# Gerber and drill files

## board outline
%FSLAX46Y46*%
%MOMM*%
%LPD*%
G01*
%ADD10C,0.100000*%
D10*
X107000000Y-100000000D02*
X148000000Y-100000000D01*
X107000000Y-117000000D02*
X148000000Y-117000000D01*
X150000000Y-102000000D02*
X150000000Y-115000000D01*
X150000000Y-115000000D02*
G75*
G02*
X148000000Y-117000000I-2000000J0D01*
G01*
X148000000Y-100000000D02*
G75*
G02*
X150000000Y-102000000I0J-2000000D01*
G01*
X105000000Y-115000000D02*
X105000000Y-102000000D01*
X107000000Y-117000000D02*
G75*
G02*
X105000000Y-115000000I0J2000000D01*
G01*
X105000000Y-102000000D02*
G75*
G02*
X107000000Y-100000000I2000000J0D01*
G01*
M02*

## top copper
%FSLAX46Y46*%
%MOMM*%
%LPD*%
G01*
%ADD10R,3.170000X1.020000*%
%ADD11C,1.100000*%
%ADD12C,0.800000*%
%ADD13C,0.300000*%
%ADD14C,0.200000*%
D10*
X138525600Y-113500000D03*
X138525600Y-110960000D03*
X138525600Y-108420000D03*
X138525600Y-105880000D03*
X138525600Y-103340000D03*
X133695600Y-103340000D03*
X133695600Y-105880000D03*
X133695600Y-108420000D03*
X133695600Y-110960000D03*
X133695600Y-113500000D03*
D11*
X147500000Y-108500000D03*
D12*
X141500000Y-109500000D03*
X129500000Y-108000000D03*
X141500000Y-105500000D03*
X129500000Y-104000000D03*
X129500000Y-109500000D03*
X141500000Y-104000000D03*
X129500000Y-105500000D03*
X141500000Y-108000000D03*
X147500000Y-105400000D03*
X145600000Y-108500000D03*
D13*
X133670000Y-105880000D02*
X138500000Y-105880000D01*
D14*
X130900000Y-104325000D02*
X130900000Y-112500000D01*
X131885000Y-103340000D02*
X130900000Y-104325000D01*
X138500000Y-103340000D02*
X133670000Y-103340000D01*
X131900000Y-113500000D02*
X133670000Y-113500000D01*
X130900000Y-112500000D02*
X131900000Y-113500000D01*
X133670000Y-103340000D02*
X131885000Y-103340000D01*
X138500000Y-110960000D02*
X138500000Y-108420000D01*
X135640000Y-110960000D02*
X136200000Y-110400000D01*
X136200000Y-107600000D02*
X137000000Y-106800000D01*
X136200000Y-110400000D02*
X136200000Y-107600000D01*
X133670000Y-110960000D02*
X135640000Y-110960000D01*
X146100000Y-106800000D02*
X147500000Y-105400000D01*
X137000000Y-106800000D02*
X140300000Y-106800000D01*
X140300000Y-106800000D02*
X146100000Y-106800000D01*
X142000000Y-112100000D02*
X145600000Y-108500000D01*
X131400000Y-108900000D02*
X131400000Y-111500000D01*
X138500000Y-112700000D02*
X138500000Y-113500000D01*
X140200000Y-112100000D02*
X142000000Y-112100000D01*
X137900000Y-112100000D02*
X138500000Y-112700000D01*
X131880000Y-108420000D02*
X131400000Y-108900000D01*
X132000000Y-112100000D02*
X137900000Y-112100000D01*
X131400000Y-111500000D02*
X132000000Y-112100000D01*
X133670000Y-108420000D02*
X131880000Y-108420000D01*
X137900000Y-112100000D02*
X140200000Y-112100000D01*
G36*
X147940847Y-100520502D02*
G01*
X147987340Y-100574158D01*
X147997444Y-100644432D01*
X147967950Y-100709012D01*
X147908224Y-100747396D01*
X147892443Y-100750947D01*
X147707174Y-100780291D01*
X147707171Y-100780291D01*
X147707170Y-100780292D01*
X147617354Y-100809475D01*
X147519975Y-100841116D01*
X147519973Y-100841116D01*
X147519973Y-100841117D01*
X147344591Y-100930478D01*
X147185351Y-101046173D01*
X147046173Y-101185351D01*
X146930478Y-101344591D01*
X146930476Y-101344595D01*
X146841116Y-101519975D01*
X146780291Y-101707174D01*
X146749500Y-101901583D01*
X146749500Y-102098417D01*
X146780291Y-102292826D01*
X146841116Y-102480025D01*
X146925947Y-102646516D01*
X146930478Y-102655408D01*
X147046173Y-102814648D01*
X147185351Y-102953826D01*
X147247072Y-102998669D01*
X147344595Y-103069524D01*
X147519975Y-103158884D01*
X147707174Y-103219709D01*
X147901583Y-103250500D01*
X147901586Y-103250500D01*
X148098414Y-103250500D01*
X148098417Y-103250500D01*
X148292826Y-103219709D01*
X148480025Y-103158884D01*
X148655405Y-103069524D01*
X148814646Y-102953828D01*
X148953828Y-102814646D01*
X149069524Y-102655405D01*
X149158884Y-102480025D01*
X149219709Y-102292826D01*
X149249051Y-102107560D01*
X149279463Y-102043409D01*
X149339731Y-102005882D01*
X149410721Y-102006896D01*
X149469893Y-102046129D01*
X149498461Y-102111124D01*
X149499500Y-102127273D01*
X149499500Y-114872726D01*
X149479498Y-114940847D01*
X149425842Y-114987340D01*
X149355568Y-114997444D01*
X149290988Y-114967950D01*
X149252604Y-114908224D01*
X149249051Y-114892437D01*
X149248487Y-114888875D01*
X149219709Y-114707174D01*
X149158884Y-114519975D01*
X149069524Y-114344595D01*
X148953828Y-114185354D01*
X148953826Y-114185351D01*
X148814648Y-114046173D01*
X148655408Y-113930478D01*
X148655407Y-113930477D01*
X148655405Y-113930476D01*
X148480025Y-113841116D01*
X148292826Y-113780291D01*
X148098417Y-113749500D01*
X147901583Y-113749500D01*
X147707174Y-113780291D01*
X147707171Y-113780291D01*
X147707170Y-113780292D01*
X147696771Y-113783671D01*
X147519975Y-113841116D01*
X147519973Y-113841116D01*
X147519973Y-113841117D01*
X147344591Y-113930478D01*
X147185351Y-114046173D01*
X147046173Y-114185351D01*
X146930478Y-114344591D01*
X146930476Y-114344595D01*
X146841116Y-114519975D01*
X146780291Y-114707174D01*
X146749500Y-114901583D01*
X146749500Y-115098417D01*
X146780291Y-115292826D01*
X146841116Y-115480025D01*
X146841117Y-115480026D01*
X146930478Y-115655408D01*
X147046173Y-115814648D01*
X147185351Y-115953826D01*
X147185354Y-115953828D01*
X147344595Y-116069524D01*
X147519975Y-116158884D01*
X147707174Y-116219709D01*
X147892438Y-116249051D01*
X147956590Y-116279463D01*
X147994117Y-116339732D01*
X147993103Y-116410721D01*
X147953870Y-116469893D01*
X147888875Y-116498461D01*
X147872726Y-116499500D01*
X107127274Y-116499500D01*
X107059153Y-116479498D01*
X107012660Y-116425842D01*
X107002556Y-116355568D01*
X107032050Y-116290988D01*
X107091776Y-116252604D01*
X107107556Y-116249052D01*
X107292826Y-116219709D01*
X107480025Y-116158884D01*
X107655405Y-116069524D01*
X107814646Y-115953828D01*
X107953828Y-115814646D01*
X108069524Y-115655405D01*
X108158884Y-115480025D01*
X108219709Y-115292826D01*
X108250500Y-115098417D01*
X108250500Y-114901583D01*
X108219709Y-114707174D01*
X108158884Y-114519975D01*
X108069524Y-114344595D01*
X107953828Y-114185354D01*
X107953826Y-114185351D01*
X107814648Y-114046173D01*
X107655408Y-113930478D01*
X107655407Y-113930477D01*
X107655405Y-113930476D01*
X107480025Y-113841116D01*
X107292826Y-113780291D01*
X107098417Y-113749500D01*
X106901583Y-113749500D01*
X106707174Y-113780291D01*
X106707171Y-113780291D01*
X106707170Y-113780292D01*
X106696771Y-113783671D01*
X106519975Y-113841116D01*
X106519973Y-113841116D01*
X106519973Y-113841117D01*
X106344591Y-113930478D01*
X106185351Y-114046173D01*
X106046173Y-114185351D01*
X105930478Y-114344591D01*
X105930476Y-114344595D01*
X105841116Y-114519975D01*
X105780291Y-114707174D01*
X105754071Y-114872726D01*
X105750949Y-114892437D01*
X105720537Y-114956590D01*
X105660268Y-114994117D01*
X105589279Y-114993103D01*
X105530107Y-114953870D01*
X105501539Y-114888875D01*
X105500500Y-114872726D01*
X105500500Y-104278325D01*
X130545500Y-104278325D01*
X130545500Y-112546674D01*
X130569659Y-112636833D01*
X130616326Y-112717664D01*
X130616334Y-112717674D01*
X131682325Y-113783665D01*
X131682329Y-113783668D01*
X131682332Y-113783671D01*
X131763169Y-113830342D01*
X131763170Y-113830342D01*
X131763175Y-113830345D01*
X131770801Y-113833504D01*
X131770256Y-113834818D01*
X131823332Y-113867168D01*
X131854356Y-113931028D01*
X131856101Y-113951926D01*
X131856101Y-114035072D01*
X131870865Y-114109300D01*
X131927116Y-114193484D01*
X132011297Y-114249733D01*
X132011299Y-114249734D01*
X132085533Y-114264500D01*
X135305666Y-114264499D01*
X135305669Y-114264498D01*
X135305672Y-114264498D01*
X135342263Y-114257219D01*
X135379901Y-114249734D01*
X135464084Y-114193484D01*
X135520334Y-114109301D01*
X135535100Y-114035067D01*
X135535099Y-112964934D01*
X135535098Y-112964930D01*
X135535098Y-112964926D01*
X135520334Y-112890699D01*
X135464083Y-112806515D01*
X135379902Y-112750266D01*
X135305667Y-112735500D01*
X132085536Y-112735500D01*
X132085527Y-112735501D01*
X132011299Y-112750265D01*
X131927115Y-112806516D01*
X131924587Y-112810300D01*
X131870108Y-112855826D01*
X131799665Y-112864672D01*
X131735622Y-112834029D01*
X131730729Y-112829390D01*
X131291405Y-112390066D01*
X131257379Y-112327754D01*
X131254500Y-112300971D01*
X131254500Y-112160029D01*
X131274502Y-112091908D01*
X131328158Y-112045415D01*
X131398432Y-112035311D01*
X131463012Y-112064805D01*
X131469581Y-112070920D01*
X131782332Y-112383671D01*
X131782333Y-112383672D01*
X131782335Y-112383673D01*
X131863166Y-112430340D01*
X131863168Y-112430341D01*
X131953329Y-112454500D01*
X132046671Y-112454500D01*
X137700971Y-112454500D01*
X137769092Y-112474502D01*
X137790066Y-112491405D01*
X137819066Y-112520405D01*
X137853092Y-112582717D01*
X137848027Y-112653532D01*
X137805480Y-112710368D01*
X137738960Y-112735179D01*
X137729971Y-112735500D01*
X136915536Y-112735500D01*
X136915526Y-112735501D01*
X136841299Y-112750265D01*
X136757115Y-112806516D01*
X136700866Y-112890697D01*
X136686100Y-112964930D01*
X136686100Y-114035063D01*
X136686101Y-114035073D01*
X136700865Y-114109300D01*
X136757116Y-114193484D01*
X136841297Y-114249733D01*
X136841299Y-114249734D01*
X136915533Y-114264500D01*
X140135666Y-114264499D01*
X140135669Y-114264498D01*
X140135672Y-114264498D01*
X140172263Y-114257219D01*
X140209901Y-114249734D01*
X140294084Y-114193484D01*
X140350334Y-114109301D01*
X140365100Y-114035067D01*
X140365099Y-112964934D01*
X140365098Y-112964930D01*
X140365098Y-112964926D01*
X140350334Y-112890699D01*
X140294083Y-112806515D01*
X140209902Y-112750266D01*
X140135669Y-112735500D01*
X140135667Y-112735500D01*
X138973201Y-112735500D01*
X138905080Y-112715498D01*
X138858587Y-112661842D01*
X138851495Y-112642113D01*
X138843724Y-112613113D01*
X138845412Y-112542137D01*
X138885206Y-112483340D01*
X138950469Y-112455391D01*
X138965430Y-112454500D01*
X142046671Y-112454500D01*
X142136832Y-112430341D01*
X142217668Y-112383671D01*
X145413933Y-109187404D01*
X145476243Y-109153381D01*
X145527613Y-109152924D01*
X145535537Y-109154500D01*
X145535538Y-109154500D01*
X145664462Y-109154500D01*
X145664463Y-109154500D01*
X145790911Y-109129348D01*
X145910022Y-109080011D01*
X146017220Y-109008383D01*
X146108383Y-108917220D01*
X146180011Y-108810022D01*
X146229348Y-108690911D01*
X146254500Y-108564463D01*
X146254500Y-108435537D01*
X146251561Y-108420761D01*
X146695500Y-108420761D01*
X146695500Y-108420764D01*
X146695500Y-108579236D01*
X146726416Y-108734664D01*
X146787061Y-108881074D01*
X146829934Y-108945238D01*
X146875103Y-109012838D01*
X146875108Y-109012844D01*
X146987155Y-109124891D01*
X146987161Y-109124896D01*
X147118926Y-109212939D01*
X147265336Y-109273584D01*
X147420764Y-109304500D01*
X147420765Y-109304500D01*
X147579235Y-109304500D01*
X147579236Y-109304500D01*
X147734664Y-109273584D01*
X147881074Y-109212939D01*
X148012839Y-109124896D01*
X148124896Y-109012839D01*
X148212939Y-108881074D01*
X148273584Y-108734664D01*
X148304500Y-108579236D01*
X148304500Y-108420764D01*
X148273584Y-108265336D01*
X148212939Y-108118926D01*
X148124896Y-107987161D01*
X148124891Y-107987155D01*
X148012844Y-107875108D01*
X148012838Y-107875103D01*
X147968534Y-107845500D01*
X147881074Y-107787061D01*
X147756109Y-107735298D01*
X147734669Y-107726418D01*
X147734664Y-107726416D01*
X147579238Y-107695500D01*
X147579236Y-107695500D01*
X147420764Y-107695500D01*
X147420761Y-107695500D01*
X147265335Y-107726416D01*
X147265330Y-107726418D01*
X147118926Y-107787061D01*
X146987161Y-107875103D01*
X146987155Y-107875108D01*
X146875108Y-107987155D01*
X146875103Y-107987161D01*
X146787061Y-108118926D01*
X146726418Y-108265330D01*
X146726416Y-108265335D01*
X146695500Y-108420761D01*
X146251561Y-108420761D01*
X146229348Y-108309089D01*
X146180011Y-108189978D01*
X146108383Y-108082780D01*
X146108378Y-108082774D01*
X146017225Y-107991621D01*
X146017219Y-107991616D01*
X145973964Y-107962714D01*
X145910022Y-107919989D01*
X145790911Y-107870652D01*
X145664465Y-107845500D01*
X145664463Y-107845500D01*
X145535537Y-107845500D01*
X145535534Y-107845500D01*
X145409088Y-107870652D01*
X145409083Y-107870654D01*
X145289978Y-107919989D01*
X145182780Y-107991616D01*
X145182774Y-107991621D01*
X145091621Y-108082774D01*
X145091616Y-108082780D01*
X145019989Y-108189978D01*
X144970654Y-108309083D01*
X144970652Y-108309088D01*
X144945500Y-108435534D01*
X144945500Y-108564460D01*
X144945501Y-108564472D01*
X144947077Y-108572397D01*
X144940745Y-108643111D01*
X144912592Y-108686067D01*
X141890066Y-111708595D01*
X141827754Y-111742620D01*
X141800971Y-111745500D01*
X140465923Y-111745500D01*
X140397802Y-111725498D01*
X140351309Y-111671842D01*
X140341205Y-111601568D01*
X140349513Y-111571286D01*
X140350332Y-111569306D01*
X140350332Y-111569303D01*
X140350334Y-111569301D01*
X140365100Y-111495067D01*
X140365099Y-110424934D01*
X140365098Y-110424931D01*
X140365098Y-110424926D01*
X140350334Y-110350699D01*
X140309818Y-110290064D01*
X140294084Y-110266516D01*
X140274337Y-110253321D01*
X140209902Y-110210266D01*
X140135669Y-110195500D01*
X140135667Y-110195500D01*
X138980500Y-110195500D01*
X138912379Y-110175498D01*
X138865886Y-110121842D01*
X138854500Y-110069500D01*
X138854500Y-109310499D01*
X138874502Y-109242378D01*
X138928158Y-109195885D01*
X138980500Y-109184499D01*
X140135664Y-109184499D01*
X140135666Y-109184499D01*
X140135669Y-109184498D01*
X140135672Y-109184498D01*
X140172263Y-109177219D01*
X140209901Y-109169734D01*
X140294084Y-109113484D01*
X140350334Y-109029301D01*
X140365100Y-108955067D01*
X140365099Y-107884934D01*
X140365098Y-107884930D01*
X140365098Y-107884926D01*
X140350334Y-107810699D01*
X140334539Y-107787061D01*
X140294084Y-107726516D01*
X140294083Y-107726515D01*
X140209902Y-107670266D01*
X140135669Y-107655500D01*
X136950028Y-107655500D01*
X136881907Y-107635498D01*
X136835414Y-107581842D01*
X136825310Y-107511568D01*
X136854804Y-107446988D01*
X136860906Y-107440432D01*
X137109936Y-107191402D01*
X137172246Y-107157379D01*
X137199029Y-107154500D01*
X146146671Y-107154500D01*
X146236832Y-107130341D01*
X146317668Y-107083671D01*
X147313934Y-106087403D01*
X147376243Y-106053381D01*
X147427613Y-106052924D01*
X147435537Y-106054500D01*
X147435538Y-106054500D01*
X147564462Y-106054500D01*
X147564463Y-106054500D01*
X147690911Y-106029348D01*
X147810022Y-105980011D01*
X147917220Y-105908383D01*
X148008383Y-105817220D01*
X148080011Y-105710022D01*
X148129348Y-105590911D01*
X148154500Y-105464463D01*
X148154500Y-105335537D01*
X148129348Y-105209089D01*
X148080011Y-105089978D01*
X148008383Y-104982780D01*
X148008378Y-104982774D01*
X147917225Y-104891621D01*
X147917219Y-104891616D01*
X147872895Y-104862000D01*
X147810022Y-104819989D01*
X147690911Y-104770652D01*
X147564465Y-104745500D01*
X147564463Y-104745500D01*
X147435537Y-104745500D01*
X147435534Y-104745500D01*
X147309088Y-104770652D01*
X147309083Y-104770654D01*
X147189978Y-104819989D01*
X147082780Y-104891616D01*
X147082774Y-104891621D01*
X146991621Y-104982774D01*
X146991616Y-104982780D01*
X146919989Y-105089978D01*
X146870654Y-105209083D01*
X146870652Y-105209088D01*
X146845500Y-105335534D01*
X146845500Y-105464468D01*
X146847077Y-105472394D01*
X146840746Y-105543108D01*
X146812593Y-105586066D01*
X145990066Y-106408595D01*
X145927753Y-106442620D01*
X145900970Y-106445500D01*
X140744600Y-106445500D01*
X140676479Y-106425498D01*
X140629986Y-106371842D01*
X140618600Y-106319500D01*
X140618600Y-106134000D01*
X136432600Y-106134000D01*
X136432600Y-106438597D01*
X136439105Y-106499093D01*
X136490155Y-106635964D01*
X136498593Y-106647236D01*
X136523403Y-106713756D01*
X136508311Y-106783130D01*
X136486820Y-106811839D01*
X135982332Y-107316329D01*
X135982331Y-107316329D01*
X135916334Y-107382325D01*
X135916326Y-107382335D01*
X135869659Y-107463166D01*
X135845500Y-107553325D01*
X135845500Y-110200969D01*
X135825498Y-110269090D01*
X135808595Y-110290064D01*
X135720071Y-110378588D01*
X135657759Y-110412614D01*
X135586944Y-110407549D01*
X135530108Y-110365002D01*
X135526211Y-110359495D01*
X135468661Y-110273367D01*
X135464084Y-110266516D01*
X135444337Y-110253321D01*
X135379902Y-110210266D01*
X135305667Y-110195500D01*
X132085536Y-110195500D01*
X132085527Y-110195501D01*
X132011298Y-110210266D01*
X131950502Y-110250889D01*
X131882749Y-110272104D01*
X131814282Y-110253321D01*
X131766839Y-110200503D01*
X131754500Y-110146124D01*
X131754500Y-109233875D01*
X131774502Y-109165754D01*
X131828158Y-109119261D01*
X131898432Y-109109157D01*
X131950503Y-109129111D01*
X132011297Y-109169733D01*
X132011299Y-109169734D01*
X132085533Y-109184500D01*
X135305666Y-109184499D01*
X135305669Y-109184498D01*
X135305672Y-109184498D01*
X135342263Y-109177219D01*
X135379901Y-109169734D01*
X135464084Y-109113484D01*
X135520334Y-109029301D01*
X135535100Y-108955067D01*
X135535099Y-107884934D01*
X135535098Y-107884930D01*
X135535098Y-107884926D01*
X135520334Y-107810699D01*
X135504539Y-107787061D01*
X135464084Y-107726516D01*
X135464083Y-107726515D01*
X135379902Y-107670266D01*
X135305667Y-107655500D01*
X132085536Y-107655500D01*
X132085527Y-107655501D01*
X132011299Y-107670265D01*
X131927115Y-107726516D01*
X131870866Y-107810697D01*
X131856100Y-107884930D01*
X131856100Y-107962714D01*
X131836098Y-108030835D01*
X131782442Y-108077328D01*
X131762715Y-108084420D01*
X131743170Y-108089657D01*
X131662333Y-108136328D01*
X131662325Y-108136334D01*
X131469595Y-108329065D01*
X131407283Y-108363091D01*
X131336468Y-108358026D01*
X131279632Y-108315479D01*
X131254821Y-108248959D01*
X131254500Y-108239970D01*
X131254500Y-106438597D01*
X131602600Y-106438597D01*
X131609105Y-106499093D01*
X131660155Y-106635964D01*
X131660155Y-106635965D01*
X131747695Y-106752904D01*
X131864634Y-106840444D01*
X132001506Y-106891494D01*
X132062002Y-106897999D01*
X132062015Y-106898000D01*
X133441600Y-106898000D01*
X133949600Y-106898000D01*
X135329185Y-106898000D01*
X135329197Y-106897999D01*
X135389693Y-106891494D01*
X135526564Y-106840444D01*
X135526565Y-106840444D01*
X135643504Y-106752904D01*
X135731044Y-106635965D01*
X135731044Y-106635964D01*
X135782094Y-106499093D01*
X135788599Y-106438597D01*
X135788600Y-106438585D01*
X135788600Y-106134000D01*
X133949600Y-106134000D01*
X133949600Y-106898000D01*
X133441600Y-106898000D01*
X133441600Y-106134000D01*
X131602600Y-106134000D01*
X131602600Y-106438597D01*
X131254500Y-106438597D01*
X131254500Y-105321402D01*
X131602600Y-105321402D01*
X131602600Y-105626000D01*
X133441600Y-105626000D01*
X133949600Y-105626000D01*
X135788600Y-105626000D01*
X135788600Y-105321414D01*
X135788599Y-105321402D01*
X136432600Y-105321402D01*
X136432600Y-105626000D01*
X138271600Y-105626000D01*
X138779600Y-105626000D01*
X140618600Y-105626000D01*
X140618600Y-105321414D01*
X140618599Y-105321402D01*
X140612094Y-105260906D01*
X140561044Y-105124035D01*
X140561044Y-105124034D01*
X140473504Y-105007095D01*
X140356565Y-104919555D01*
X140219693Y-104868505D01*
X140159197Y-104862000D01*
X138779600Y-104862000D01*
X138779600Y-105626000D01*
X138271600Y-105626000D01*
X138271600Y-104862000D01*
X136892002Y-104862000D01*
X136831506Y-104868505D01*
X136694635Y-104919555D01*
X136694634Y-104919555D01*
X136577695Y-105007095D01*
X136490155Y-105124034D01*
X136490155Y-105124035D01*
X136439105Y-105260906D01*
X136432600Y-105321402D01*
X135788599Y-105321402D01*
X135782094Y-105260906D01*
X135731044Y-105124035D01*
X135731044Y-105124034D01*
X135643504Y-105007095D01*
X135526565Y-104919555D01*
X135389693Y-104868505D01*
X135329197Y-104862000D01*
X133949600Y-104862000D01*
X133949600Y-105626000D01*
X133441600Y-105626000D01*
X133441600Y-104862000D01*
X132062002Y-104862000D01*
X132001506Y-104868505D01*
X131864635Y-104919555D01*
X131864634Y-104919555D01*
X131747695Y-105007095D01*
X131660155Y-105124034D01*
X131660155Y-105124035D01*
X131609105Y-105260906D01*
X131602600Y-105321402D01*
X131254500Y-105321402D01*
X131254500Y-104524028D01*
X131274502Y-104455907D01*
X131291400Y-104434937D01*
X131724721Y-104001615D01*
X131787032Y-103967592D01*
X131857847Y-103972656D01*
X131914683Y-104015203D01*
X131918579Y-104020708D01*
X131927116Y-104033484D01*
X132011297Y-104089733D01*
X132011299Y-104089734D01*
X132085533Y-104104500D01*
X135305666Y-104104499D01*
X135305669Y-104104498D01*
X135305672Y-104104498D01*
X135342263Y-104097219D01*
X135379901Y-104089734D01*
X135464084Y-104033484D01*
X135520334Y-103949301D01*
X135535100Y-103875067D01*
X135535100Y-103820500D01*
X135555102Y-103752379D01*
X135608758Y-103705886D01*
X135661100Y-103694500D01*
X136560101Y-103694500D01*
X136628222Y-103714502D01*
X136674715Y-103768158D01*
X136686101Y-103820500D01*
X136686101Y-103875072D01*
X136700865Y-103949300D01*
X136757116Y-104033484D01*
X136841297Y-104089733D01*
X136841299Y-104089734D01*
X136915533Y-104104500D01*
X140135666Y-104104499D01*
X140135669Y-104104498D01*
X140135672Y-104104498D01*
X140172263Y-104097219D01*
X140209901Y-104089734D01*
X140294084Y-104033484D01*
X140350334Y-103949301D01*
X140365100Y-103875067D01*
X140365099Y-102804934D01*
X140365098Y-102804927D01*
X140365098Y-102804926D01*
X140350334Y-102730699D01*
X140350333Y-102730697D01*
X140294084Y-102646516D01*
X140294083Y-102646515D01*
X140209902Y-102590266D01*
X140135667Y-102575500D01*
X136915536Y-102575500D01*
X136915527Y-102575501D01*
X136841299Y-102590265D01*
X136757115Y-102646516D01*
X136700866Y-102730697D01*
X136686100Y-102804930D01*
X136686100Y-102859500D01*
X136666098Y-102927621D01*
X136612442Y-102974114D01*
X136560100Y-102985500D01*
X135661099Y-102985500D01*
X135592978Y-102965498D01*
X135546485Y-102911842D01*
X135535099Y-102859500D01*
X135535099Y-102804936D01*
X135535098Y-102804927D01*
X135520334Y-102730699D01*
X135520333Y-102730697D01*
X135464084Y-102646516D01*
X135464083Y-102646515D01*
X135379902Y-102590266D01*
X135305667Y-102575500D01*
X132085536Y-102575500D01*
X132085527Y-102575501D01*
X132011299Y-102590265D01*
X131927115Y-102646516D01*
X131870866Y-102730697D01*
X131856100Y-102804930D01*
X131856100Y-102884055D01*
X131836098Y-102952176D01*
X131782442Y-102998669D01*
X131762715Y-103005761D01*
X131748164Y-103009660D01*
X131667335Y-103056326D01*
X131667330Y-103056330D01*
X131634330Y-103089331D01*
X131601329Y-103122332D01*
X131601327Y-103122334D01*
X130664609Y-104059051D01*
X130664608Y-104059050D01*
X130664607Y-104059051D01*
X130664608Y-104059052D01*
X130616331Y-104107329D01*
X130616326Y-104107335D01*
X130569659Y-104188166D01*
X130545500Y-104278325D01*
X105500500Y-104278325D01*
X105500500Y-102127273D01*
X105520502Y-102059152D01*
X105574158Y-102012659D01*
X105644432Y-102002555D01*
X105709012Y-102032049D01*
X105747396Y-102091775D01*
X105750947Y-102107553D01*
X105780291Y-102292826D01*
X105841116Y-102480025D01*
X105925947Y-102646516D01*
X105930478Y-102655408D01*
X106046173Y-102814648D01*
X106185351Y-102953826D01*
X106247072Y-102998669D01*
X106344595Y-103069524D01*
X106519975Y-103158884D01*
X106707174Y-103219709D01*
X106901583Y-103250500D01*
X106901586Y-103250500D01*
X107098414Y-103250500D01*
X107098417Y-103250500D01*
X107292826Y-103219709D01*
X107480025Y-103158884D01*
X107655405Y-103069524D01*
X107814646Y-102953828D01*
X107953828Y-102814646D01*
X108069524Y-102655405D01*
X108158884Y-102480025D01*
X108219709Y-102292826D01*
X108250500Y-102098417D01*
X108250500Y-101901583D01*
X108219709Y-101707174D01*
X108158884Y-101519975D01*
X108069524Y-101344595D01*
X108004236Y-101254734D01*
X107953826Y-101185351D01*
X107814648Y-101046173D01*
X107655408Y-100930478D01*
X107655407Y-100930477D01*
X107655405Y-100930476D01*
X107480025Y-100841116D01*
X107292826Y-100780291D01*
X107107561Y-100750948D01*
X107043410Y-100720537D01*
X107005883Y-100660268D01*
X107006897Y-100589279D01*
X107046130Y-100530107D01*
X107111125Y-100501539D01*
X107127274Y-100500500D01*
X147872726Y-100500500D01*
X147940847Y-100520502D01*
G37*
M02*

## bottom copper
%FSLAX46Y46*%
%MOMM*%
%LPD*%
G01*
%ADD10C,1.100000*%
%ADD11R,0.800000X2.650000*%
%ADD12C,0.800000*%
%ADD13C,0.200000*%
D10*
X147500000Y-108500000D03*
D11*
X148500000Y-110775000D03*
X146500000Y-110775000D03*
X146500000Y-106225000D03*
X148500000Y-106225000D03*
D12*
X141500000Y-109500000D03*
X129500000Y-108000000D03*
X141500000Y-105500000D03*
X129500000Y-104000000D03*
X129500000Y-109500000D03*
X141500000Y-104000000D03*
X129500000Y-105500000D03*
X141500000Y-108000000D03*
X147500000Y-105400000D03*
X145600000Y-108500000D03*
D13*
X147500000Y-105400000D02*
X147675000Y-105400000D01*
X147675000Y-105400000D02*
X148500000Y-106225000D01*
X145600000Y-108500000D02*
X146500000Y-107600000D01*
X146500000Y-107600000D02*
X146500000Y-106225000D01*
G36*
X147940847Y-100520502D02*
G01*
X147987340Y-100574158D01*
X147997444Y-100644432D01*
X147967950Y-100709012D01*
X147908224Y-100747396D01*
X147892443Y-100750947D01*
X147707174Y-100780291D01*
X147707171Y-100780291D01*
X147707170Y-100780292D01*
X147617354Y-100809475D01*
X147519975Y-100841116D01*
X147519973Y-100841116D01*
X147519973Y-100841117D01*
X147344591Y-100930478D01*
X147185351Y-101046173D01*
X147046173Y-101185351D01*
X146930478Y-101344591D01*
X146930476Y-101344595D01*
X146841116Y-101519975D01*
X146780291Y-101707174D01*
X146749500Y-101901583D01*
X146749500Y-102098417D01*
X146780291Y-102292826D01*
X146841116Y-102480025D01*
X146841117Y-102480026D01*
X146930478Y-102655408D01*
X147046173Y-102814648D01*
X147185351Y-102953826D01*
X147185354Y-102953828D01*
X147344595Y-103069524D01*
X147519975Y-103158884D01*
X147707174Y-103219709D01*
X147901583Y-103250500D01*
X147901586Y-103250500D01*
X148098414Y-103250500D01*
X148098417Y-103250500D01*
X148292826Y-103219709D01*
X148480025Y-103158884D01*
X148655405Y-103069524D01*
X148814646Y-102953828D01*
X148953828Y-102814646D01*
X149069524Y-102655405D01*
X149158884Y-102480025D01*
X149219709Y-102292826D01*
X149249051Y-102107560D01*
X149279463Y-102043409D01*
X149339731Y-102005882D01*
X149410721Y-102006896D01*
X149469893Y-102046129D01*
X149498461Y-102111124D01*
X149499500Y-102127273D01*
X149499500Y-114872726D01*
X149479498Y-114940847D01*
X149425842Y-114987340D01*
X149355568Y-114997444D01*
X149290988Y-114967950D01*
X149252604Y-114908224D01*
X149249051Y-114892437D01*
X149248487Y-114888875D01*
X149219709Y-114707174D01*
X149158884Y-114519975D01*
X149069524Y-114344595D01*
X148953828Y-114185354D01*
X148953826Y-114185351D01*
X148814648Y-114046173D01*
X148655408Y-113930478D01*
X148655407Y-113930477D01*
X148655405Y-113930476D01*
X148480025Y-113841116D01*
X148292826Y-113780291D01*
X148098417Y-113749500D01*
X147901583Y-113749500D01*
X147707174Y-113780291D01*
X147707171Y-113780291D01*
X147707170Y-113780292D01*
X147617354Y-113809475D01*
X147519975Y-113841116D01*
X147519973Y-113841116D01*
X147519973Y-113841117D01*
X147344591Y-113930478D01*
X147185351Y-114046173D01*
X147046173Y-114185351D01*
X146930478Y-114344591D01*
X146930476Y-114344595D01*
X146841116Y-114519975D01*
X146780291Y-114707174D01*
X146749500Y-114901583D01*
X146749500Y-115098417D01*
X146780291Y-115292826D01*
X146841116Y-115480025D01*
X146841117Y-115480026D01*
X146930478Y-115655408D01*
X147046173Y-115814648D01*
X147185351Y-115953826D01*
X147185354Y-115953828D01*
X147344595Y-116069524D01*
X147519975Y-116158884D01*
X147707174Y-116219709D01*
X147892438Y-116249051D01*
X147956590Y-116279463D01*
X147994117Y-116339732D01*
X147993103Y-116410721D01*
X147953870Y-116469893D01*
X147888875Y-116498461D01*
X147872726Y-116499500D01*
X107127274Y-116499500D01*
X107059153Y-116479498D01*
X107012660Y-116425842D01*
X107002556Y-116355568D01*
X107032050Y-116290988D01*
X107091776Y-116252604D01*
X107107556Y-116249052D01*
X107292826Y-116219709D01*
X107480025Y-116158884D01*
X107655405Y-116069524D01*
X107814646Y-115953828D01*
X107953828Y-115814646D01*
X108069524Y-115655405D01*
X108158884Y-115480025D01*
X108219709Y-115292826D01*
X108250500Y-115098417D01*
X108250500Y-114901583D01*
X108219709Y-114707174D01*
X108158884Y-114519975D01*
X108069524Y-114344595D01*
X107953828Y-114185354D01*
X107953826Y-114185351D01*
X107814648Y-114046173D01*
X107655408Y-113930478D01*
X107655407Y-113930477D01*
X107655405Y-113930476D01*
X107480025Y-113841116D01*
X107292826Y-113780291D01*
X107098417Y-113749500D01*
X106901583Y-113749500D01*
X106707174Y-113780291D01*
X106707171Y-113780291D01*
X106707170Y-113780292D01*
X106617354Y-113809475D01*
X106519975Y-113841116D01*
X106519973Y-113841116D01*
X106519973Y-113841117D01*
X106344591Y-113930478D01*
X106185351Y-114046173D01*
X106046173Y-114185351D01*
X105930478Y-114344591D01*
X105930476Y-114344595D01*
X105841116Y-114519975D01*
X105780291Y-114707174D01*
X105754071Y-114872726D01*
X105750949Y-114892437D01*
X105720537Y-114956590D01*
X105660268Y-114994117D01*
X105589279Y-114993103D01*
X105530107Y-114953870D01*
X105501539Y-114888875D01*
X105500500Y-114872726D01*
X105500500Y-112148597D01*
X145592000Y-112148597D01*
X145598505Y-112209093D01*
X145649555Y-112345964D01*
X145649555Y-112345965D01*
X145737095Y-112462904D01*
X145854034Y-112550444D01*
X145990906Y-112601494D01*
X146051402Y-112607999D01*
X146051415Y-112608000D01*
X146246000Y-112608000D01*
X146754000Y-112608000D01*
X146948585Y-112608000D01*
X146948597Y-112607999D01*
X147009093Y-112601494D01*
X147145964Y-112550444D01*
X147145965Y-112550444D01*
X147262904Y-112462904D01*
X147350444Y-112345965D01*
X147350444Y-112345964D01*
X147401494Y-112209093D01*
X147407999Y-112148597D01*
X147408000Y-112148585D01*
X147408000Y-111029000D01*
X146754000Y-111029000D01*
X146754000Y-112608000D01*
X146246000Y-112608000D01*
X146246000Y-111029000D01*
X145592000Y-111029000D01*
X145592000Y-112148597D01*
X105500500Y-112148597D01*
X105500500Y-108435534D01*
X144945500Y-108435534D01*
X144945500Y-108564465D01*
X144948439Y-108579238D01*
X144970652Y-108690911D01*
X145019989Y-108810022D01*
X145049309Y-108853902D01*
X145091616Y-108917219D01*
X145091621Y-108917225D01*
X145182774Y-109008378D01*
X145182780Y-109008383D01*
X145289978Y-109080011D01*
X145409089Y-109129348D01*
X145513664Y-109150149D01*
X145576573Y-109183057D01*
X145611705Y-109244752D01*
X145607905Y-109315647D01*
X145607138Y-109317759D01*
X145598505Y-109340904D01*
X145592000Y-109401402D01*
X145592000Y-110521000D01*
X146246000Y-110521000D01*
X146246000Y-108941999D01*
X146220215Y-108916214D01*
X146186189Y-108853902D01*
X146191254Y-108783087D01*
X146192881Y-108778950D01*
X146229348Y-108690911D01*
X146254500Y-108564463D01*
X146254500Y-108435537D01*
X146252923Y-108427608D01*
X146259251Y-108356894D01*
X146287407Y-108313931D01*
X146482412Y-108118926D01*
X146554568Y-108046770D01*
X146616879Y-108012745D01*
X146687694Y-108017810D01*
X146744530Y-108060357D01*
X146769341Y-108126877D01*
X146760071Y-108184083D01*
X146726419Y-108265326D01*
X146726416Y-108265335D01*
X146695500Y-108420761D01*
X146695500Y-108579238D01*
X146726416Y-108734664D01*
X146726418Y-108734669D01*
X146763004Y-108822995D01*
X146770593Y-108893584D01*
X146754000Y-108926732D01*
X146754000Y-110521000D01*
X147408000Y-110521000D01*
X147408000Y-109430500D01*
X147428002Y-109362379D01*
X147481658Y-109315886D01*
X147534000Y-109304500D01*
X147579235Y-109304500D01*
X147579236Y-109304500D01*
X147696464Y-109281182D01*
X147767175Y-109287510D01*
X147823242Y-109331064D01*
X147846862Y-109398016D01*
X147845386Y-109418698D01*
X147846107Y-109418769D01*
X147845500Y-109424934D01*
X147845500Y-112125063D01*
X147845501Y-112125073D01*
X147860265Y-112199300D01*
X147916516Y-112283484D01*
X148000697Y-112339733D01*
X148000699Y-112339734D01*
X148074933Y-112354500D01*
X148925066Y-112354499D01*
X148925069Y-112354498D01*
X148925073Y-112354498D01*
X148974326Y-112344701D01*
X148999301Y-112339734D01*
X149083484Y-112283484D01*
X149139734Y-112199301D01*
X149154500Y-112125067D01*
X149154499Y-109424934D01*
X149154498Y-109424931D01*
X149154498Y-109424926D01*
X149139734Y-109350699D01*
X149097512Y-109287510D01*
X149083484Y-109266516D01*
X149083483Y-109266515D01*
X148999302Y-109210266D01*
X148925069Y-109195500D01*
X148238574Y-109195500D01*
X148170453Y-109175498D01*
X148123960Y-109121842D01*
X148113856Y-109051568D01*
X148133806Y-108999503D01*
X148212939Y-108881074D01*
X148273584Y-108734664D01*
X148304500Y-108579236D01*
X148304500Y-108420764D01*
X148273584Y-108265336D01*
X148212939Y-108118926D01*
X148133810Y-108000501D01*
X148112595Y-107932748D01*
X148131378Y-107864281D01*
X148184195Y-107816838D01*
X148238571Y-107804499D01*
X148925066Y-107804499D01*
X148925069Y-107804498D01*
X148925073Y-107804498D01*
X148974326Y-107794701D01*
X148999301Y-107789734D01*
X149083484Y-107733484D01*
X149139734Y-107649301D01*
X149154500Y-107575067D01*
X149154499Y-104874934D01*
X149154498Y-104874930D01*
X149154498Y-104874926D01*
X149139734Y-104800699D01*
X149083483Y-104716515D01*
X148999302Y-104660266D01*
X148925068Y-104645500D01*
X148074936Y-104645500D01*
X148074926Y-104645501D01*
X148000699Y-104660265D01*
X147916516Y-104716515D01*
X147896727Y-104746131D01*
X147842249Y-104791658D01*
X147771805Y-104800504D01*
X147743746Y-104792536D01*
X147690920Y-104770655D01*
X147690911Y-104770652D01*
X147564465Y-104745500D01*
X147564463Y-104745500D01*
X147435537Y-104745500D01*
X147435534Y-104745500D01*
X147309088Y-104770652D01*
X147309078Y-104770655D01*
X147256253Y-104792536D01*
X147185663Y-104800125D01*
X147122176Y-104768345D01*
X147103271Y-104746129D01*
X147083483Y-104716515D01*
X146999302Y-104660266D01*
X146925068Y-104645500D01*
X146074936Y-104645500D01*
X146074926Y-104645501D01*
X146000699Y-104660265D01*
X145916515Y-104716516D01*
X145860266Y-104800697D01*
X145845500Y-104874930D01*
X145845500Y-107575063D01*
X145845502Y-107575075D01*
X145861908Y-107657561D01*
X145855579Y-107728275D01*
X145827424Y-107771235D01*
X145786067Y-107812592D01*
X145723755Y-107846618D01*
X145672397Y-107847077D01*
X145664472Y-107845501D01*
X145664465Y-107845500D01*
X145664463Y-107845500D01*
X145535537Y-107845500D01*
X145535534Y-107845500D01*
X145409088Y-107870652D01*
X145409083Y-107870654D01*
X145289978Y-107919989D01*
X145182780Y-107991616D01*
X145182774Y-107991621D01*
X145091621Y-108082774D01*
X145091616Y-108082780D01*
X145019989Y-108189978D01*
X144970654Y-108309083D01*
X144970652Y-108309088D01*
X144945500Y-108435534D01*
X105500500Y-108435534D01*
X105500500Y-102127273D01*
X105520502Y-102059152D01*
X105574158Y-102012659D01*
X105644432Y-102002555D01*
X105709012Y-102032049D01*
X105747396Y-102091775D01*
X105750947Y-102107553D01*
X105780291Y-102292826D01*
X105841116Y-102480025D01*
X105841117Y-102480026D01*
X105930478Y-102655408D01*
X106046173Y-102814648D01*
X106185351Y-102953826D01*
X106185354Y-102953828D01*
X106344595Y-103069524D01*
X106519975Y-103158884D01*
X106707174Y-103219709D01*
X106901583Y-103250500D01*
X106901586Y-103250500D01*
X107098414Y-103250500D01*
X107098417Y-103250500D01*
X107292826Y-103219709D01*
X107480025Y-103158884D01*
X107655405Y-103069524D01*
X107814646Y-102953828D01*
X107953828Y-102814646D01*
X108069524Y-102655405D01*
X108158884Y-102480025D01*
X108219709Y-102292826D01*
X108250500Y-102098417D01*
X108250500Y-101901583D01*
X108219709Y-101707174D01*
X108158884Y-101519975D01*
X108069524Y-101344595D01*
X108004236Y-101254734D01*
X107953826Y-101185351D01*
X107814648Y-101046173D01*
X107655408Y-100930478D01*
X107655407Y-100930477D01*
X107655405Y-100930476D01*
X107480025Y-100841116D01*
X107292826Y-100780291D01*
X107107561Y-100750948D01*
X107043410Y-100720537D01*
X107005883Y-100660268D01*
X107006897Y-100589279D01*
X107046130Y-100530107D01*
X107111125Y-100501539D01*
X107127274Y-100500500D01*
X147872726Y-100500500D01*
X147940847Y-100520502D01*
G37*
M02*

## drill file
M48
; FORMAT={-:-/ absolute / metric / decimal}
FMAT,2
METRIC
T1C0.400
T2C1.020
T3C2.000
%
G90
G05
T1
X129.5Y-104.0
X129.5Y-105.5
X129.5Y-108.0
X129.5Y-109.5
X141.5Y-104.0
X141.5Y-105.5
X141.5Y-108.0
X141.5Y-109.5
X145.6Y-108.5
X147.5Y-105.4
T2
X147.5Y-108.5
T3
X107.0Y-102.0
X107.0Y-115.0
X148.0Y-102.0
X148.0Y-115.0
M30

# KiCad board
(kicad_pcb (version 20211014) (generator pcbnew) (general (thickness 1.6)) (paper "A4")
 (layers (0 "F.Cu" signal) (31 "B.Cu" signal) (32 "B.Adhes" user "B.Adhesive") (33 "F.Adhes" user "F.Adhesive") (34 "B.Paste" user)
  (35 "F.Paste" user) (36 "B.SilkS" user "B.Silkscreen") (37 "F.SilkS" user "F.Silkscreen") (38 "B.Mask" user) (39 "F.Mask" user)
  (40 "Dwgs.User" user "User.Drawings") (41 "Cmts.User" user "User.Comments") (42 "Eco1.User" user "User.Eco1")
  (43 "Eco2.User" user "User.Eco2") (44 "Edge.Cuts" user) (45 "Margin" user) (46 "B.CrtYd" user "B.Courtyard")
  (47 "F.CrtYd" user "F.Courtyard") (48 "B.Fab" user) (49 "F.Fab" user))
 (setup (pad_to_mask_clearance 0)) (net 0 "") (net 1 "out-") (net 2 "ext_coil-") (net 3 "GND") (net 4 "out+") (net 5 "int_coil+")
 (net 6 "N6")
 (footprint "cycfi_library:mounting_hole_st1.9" (layer "F.Cu") (at 107 102)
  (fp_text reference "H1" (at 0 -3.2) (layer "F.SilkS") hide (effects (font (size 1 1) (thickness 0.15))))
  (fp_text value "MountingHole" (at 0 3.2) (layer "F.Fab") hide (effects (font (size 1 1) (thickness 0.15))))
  (pad "" np_thru_hole circle locked (at 0 0) (size 2 2) (drill 2) (layers *.Cu *.Mask)))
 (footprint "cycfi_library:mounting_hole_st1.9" (layer "F.Cu") (at 107 115)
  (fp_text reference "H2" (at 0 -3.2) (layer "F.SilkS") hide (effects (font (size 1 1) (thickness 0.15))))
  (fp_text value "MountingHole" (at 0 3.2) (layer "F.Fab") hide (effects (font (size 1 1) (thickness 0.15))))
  (pad "" np_thru_hole circle locked (at 0 0) (size 2 2) (drill 2) (layers *.Cu *.Mask)))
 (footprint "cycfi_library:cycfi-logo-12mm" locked (layer "F.Cu") (at 109.75 108.5 -90)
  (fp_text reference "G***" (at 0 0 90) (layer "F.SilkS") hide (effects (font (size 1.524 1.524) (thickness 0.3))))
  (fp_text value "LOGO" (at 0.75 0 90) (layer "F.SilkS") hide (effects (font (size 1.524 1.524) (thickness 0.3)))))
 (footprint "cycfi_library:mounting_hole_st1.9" (layer "F.Cu") (at 148 102)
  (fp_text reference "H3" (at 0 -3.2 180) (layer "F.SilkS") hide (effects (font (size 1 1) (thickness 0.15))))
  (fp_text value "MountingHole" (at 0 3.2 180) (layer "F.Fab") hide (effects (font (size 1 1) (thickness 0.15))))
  (pad "" np_thru_hole circle locked (at 0 0) (size 2 2) (drill 2) (layers *.Cu *.Mask)))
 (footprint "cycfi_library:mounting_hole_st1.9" (layer "F.Cu") (at 148 115)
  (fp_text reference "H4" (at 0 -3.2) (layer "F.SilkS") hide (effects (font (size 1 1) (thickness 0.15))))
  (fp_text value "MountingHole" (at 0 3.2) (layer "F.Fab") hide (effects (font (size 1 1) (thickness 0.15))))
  (pad "" np_thru_hole circle locked (at 0 0) (size 2 2) (drill 2) (layers *.Cu *.Mask)))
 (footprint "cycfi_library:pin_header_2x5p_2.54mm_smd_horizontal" (layer "F.Cu") (at 136.1 108.42 180)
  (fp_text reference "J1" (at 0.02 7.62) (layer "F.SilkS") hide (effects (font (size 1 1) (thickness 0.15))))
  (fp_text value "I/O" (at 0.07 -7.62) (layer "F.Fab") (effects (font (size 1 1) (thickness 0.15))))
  (pad "1" smd rect (at -2.4256 -5.08 180) (size 3.17 1.02) (layers "F.Cu" "F.Paste" "F.Mask") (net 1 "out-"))
  (pad "2" smd rect (at -2.4256 -2.54 180) (size 3.17 1.02) (layers "F.Cu" "F.Paste" "F.Mask") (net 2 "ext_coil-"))
  (pad "3" smd rect (at -2.4256 0 180) (size 3.17 1.02) (layers "F.Cu" "F.Paste" "F.Mask") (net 2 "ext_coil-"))
  (pad "4" smd rect (at -2.4256 2.54 180) (size 3.17 1.02) (layers "F.Cu" "F.Paste" "F.Mask") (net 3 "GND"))
  (pad "5" smd rect (at -2.4256 5.08 180) (size 3.17 1.02) (layers "F.Cu" "F.Paste" "F.Mask") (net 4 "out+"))
  (pad "6" smd rect (at 2.4044 5.08 180) (size 3.17 1.02) (layers "F.Cu" "F.Paste" "F.Mask") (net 4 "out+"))
  (pad "7" smd rect (at 2.4044 2.54 180) (size 3.17 1.02) (layers "F.Cu" "F.Paste" "F.Mask") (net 3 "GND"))
  (pad "8" smd rect (at 2.4044 0 180) (size 3.17 1.02) (layers "F.Cu" "F.Paste" "F.Mask") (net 1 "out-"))
  (pad "9" smd rect (at 2.4044 -2.54 180) (size 3.17 1.02) (layers "F.Cu" "F.Paste" "F.Mask") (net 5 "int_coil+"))
  (pad "10" smd rect (at 2.4044 -5.08 180) (size 3.17 1.02) (layers "F.Cu" "F.Paste" "F.Mask") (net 4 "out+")))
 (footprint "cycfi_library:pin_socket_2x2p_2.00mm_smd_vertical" (layer "B.Cu") (at 147.5 108.5 90)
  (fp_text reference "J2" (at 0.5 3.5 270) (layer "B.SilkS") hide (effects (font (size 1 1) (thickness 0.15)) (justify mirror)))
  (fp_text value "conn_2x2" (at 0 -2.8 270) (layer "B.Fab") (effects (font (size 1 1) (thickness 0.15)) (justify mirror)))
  (pad "" np_thru_hole circle (at 0 0 90) (size 1.1 1.1) (drill 1.02) (layers F&B.Cu *.Mask))
  (pad "1" smd rect (at -2.275 1 90) (size 2.65 0.8) (layers "B.Cu" "B.Paste" "B.Mask") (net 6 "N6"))
  (pad "2" smd rect (at -2.275 -1 90) (size 2.65 0.8) (layers "B.Cu" "B.Paste" "B.Mask") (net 3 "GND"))
  (pad "3" smd rect (at 2.275 -1 90) (size 2.65 0.8) (layers "B.Cu" "B.Paste" "B.Mask") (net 1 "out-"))
  (pad "4" smd rect (at 2.275 1 90) (size 2.65 0.8) (layers "B.Cu" "B.Paste" "B.Mask") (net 5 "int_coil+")))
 (gr_line (start 107 100) (end 148 100) (layer "Edge.Cuts") (width 0.1))
 (gr_line (start 107 117) (end 148 117) (layer "Edge.Cuts") (width 0.1))
 (gr_line (start 150 102) (end 150 115) (layer "Edge.Cuts") (width 0.1))
 (gr_arc (start 150 115) (mid 149.414214 116.414214) (end 148 117) (layer "Edge.Cuts") (width 0.1))
 (gr_arc (start 148 100) (mid 149.414214 100.585786) (end 150 102) (layer "Edge.Cuts") (width 0.1))
 (gr_line (start 105 115) (end 105 102) (layer "Edge.Cuts") (width 0.1))
 (gr_arc (start 107 117) (mid 105.585786 116.414214) (end 105 115) (layer "Edge.Cuts") (width 0.1))
 (gr_arc (start 105 102) (mid 105.585786 100.585786) (end 107 100) (layer "Edge.Cuts") (width 0.1))
 (segment (start 133.67 105.88) (end 138.5 105.88) (width 0.3) (layer "F.Cu") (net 3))
 (via (at 141.5 109.5) (size 0.8) (drill 0.4) (layers "F.Cu" "B.Cu") (free) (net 3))
 (via (at 129.5 108) (size 0.8) (drill 0.4) (layers "F.Cu" "B.Cu") (free) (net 3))
 (via (at 141.5 105.5) (size 0.8) (drill 0.4) (layers "F.Cu" "B.Cu") (free) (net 3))
 (via (at 129.5 104) (size 0.8) (drill 0.4) (layers "F.Cu" "B.Cu") (free) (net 3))
 (via (at 129.5 109.5) (size 0.8) (drill 0.4) (layers "F.Cu" "B.Cu") (free) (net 3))
 (via (at 141.5 104) (size 0.8) (drill 0.4) (layers "F.Cu" "B.Cu") (free) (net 3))
 (via (at 129.5 105.5) (size 0.8) (drill 0.4) (layers "F.Cu" "B.Cu") (free) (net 3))
 (via (at 141.5 108) (size 0.8) (drill 0.4) (layers "F.Cu" "B.Cu") (free) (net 3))
 (segment (start 130.9 104.325) (end 130.9 112.5) (width 0.2) (layer "F.Cu") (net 4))
 (segment (start 131.885 103.34) (end 130.9 104.325) (width 0.2) (layer "F.Cu") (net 4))
 (segment (start 138.5 103.34) (end 133.67 103.34) (width 0.2) (layer "F.Cu") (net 4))
 (segment (start 131.9 113.5) (end 133.67 113.5) (width 0.2) (layer "F.Cu") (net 4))
 (segment (start 130.9 112.5) (end 131.9 113.5) (width 0.2) (layer "F.Cu") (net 4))
 (segment (start 133.67 103.34) (end 131.885 103.34) (width 0.2) (layer "F.Cu") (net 4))
 (segment (start 138.5 110.96) (end 138.5 108.42) (width 0.2) (layer "F.Cu") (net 2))
 (segment (start 135.64 110.96) (end 136.2 110.4) (width 0.2) (layer "F.Cu") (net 5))
 (segment (start 136.2 107.6) (end 137 106.8) (width 0.2) (layer "F.Cu") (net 5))
 (segment (start 136.2 110.4) (end 136.2 107.6) (width 0.2) (layer "F.Cu") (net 5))
 (segment (start 133.67 110.96) (end 135.64 110.96) (width 0.2) (layer "F.Cu") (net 5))
 (segment (start 146.1 106.8) (end 147.5 105.4) (width 0.2) (layer "F.Cu") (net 5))
 (segment (start 137 106.8) (end 140.3 106.8) (width 0.2) (layer "F.Cu") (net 5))
 (segment (start 140.3 106.8) (end 146.1 106.8) (width 0.2) (layer "F.Cu") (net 5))
 (via (at 147.5 105.4) (size 0.8) (drill 0.4) (layers "F.Cu" "B.Cu") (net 5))
 (segment (start 147.5 105.4) (end 147.675 105.4) (width 0.2) (layer "B.Cu") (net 5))
 (segment (start 147.675 105.4) (end 148.5 106.225) (width 0.2) (layer "B.Cu") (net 5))
 (segment (start 142 112.1) (end 145.6 108.5) (width 0.2) (layer "F.Cu") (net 1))
 (segment (start 131.4 108.9) (end 131.4 111.5) (width 0.2) (layer "F.Cu") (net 1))
 (segment (start 138.5 112.7) (end 138.5 113.5) (width 0.2) (layer "F.Cu") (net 1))
 (segment (start 140.2 112.1) (end 142 112.1) (width 0.2) (layer "F.Cu") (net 1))
 (segment (start 137.9 112.1) (end 138.5 112.7) (width 0.2) (layer "F.Cu") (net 1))
 (segment (start 131.88 108.42) (end 131.4 108.9) (width 0.2) (layer "F.Cu") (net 1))
 (segment (start 132 112.1) (end 137.9 112.1) (width 0.2) (layer "F.Cu") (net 1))
 (segment (start 131.4 111.5) (end 132 112.1) (width 0.2) (layer "F.Cu") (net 1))
 (segment (start 133.67 108.42) (end 131.88 108.42) (width 0.2) (layer "F.Cu") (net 1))
 (segment (start 137.9 112.1) (end 140.2 112.1) (width 0.2) (layer "F.Cu") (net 1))
 (via (at 145.6 108.5) (size 0.8) (drill 0.4) (layers "F.Cu" "B.Cu") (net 1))
 (segment (start 145.6 108.5) (end 146.5 107.6) (width 0.2) (layer "B.Cu") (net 1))
 (segment (start 146.5 107.6) (end 146.5 106.225) (width 0.2) (layer "B.Cu") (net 1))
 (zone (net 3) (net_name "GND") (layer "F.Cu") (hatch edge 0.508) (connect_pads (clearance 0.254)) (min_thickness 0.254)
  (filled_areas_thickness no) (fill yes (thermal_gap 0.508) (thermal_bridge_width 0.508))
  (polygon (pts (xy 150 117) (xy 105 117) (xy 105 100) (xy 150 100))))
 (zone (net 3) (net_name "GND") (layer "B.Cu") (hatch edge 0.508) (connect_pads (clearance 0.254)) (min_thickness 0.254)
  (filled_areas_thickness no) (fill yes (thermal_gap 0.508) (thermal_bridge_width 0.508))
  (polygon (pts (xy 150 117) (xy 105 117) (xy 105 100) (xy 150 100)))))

